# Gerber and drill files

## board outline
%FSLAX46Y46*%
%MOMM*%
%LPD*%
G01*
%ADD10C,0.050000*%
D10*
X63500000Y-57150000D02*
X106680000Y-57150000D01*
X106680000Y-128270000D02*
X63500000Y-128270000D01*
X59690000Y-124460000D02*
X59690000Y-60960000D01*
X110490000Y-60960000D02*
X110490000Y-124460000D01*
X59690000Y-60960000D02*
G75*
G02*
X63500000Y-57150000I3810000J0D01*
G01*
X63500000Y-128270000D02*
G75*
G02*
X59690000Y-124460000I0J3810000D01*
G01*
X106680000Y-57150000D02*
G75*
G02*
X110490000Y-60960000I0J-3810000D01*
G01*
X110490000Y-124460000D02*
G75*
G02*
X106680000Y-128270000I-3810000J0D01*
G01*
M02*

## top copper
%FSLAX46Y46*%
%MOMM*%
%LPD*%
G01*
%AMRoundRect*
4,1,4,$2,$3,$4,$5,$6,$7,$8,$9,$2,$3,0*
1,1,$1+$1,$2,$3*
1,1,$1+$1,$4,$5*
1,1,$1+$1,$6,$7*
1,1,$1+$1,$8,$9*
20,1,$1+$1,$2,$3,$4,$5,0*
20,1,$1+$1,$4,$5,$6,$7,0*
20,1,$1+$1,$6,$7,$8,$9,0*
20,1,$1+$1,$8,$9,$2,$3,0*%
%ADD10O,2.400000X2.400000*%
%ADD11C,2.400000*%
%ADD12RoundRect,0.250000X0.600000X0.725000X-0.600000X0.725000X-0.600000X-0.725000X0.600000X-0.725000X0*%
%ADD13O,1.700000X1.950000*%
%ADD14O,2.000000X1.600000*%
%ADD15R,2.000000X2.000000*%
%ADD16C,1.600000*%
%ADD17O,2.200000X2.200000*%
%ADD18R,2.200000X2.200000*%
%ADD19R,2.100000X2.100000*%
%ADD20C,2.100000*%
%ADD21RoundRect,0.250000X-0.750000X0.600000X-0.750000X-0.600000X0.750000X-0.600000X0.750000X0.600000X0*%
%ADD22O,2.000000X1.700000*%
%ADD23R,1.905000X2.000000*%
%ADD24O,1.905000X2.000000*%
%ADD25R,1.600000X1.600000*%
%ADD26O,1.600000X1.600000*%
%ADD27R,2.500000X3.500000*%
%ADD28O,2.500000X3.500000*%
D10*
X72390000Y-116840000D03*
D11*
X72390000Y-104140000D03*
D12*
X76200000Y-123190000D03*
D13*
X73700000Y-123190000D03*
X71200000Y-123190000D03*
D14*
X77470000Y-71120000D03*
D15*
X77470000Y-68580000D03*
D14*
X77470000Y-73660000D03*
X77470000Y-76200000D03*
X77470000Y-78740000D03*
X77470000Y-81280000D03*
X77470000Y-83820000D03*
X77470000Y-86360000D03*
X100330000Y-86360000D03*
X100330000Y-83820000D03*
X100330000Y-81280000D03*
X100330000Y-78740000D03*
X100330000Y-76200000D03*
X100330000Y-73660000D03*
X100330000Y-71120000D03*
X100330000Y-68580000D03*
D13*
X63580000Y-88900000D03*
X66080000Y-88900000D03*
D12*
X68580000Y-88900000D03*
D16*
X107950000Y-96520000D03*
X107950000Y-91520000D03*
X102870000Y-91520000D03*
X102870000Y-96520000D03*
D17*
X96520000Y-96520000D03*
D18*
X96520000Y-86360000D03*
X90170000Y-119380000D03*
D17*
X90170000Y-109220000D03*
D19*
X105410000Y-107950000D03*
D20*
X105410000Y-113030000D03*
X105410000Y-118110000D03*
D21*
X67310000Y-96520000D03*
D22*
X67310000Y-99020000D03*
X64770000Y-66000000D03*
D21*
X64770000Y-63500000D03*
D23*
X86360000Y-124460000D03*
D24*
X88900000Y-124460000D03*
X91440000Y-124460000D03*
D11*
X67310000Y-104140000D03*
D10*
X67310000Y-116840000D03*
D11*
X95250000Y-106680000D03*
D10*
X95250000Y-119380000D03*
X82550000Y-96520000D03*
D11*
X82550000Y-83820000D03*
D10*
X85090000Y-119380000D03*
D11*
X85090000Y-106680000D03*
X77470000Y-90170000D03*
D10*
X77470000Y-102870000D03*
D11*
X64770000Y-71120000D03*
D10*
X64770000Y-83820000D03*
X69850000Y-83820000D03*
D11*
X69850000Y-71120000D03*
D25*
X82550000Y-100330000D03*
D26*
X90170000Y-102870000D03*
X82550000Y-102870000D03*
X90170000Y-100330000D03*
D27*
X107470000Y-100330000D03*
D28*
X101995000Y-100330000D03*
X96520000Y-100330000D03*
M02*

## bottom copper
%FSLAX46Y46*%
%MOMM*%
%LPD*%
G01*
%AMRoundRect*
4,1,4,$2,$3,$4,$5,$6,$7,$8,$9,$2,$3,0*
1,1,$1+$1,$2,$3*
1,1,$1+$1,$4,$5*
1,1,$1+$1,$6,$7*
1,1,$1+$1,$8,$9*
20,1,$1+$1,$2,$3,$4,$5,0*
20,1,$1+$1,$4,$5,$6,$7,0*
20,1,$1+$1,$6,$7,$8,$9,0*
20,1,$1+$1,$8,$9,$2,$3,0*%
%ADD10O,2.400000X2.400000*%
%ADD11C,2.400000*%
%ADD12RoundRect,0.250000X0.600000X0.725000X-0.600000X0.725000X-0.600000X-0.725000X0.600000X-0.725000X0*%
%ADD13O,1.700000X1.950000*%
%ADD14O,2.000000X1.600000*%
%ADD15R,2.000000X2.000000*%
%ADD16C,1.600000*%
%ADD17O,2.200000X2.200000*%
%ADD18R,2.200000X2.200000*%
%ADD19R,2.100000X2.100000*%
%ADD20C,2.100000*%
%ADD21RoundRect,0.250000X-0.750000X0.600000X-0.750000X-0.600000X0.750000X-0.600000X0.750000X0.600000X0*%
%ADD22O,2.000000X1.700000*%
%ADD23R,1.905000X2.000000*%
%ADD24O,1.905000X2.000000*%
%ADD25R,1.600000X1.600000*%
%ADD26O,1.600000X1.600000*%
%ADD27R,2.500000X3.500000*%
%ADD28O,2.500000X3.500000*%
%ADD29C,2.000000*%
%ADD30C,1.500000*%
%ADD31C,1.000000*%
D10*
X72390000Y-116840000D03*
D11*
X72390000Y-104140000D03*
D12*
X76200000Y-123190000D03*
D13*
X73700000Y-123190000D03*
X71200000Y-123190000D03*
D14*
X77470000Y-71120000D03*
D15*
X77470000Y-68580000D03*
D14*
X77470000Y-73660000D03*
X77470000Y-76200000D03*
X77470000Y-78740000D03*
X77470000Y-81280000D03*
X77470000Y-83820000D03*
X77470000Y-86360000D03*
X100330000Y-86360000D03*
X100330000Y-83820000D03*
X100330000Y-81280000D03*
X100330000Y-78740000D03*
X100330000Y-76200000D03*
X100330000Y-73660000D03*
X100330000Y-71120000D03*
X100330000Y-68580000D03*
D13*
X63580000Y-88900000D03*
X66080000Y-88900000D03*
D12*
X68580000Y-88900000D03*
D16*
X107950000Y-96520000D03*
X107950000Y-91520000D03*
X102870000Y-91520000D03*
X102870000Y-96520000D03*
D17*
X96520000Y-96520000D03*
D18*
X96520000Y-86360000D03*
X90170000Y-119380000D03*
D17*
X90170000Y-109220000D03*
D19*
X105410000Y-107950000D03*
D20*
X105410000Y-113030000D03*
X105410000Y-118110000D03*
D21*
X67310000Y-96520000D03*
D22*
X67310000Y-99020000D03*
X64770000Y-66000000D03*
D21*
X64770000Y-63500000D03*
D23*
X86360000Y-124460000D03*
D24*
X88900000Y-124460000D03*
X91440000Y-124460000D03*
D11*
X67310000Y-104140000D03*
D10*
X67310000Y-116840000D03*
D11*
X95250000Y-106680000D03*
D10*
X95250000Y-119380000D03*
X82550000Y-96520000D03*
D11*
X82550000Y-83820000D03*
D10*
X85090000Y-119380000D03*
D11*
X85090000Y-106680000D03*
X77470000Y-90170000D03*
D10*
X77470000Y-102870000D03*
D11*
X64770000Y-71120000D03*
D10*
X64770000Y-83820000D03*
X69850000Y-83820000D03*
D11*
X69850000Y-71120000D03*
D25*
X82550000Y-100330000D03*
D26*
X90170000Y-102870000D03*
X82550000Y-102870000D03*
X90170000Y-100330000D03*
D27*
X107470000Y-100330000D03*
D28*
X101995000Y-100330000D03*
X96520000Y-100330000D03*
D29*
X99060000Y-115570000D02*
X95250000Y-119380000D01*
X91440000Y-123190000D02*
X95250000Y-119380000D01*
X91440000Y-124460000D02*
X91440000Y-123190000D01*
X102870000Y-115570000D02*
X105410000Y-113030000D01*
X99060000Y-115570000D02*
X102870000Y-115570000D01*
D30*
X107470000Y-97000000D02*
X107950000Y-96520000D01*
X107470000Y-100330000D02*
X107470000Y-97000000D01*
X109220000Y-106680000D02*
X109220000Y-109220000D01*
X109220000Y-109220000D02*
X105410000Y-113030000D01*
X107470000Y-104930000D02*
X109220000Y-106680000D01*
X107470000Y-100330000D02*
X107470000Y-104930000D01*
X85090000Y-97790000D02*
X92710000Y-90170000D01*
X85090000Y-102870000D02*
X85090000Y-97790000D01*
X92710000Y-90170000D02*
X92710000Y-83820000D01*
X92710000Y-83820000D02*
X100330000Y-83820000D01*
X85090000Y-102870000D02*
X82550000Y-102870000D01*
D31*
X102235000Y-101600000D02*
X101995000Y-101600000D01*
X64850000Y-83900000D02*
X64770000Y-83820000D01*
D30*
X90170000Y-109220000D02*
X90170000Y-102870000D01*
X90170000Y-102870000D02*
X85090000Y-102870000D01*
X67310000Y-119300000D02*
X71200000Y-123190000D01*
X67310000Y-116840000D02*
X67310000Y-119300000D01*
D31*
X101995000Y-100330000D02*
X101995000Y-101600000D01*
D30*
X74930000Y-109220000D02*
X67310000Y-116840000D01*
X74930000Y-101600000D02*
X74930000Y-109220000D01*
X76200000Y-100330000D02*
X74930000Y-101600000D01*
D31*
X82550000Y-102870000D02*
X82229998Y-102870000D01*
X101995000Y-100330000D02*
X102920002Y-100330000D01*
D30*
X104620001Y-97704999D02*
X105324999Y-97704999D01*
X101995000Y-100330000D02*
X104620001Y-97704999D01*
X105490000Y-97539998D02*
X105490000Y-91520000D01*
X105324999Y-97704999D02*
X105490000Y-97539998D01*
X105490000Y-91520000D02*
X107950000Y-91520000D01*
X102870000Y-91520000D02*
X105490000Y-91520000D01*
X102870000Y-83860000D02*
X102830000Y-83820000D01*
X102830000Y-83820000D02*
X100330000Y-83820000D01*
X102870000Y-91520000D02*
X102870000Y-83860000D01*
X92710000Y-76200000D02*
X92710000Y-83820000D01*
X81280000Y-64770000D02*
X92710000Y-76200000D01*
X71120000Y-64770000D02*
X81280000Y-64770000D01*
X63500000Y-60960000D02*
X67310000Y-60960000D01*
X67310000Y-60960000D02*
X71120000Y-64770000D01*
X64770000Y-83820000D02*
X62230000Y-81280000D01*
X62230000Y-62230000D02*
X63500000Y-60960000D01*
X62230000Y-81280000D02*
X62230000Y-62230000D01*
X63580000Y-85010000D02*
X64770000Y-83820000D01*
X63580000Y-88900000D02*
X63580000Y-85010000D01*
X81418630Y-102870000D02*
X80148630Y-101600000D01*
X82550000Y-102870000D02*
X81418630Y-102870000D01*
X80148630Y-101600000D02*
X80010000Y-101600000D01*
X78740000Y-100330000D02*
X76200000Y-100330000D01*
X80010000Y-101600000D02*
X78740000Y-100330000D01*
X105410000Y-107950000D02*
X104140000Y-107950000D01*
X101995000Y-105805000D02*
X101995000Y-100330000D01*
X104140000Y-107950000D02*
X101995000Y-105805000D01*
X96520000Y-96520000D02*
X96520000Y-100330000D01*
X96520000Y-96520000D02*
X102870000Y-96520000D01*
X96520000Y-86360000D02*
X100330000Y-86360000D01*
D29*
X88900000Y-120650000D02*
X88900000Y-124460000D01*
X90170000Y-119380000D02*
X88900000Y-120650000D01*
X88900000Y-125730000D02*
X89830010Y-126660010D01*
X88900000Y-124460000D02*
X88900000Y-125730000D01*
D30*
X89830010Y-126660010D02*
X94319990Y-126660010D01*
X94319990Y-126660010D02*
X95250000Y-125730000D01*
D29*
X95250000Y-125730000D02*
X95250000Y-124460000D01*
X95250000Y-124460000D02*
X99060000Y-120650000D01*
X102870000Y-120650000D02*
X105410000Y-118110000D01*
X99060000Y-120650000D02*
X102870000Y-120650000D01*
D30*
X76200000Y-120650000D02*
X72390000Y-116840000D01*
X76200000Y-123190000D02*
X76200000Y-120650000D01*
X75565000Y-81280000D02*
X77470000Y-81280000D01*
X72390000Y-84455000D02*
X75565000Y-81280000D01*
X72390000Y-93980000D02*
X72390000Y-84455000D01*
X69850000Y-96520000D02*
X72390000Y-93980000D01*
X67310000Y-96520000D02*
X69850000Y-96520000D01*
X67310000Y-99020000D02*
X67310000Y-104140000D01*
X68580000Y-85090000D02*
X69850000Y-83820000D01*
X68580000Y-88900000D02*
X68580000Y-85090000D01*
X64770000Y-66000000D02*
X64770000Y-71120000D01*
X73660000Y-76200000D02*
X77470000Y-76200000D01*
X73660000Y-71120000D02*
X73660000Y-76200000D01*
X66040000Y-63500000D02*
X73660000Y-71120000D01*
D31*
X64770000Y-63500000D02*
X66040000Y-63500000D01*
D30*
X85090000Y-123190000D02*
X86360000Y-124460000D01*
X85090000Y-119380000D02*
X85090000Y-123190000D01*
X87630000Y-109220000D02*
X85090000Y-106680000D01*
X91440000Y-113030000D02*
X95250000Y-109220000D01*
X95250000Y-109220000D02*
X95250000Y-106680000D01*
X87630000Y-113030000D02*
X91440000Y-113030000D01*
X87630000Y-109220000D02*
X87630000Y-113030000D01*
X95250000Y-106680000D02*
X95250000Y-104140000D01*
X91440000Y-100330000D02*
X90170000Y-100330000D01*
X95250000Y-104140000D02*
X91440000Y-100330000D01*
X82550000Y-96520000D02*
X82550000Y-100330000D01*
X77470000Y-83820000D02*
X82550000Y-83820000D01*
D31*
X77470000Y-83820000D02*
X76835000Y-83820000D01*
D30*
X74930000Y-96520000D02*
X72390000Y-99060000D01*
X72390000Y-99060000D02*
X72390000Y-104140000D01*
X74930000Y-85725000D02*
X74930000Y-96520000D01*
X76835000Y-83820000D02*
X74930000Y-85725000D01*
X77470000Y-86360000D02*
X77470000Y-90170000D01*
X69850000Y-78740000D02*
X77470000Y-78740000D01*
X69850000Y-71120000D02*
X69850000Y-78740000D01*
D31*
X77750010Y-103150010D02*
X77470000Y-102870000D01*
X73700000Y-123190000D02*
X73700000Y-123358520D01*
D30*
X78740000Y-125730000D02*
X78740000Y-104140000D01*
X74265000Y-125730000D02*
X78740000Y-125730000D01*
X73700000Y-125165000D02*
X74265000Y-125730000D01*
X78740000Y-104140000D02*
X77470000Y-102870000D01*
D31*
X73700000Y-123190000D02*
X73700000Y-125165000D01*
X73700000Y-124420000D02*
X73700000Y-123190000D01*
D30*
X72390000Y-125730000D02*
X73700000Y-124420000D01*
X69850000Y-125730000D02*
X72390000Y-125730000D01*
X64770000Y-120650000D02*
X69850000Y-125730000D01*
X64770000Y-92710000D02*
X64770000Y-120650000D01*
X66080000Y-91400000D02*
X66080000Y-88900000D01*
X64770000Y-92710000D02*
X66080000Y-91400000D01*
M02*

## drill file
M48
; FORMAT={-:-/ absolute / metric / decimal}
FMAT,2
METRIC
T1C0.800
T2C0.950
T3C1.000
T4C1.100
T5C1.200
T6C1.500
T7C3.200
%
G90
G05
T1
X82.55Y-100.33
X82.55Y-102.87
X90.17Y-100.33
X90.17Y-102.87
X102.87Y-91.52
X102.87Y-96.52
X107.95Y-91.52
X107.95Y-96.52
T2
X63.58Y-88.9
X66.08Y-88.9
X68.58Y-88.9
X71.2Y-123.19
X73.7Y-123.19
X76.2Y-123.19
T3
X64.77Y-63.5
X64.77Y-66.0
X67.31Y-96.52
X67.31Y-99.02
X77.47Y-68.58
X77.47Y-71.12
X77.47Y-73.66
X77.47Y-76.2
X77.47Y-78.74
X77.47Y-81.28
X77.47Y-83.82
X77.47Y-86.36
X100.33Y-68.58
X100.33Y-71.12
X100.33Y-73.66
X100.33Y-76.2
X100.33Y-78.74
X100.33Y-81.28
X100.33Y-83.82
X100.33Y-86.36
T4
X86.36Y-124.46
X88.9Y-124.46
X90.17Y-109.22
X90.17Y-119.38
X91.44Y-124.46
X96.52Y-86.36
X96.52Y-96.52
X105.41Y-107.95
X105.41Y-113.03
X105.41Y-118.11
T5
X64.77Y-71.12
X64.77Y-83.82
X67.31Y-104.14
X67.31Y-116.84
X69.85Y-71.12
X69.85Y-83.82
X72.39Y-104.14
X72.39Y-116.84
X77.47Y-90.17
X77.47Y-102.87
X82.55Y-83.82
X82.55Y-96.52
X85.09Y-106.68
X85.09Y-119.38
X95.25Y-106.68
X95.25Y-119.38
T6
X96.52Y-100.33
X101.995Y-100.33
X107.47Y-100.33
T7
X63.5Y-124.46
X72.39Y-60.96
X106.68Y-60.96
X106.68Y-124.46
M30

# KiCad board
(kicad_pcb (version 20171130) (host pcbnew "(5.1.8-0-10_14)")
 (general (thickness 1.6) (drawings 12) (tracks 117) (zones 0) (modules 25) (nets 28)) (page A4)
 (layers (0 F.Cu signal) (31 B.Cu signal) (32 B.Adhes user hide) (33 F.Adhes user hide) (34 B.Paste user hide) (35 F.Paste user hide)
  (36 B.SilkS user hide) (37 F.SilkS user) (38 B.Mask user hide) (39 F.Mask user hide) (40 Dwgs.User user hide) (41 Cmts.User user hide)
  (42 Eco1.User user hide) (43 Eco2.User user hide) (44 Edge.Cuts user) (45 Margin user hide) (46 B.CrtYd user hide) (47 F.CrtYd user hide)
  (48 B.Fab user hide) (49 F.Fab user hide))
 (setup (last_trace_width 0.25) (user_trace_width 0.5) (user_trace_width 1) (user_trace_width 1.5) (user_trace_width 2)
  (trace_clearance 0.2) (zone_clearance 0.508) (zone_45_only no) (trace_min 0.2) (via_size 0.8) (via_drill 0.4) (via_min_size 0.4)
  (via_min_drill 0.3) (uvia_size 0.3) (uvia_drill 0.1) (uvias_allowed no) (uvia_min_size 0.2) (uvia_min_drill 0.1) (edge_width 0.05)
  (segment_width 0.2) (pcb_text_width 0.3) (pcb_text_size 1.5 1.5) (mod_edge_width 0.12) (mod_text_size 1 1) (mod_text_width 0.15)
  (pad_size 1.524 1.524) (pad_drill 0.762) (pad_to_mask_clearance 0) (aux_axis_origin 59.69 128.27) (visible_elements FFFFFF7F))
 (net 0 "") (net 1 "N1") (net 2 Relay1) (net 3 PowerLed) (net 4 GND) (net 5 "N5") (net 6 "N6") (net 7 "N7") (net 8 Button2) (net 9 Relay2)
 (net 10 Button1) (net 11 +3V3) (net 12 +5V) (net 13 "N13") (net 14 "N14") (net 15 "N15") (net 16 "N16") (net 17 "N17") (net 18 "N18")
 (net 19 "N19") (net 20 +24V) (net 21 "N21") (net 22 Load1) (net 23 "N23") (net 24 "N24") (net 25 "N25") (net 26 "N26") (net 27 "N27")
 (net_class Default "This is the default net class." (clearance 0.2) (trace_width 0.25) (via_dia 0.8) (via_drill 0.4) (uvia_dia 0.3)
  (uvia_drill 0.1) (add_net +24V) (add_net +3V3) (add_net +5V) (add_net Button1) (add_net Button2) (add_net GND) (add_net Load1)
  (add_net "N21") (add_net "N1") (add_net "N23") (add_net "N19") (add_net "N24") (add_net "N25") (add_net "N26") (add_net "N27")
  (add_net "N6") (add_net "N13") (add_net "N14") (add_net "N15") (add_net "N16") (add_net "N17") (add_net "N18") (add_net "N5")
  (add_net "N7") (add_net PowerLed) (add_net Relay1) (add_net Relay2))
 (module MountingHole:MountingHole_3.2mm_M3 (layer F.Cu) (at 72.39 60.96 270)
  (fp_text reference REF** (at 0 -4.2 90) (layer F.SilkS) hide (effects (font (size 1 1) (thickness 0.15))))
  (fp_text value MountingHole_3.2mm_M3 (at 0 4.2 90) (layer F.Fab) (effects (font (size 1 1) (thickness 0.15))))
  (pad 1 np_thru_hole circle (at 0 0 270) (size 3.2 3.2) (drill 3.2) (layers *.Cu *.Mask)))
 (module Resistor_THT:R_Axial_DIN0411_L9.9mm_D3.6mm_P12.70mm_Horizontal (layer F.Cu) (at 72.39 104.14 270)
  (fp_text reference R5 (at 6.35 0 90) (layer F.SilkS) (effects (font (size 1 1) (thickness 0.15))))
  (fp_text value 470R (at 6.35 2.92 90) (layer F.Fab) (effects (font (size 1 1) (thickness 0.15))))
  (pad 2 thru_hole oval (at 12.7 0 270) (size 2.4 2.4) (drill 1.2) (layers *.Cu *.Mask) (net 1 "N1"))
  (pad 1 thru_hole circle (at 0 0 270) (size 2.4 2.4) (drill 1.2) (layers *.Cu *.Mask) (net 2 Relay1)))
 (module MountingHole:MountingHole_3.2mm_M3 (layer F.Cu) (at 106.68 124.46 270)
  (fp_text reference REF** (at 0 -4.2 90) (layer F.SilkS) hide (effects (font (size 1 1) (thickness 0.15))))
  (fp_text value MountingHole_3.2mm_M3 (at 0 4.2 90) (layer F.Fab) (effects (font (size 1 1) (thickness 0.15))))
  (pad 1 np_thru_hole circle (at 0 0 270) (size 3.2 3.2) (drill 3.2) (layers *.Cu *.Mask)))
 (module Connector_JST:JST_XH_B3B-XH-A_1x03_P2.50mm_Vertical (layer F.Cu) (at 76.2 123.19 180)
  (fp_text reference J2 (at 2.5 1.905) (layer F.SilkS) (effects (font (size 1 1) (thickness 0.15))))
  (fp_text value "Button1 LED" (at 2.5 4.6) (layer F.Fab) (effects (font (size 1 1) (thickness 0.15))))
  (pad 1 thru_hole roundrect (at 0 0 180) (size 1.7 1.95) (drill 0.95) (layers *.Cu *.Mask) (roundrect_rratio 0.1470588235294118)
   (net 1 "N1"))
  (pad 2 thru_hole oval (at 2.5 0 180) (size 1.7 1.95) (drill 0.95) (layers *.Cu *.Mask) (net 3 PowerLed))
  (pad 3 thru_hole oval (at 5 0 180) (size 1.7 1.95) (drill 0.95) (layers *.Cu *.Mask) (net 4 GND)))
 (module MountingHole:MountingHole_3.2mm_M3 (layer F.Cu) (at 63.5 124.46 270)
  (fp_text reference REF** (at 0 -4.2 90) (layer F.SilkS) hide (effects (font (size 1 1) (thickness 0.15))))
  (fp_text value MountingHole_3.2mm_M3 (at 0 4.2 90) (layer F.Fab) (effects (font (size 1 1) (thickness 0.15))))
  (pad 1 np_thru_hole circle (at 0 0 270) (size 3.2 3.2) (drill 3.2) (layers *.Cu *.Mask)))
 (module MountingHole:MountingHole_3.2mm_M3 (layer F.Cu) (at 106.68 60.96 270)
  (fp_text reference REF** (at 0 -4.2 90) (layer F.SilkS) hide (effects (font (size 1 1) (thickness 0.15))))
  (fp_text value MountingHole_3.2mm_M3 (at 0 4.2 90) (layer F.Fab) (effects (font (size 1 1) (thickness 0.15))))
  (pad 1 np_thru_hole circle (at 0 0 270) (size 3.2 3.2) (drill 3.2) (layers *.Cu *.Mask)))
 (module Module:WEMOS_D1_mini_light (layer F.Cu) (at 77.47 68.58)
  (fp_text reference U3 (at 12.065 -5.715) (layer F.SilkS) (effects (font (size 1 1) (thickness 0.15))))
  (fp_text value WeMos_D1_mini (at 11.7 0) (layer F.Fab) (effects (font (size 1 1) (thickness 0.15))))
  (pad 2 thru_hole oval (at 0 2.54) (size 2 1.6) (drill 1) (layers *.Cu *.Mask) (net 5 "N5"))
  (pad 1 thru_hole rect (at 0 0) (size 2 2) (drill 1) (layers *.Cu *.Mask) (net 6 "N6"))
  (pad 3 thru_hole oval (at 0 5.08) (size 2 1.6) (drill 1) (layers *.Cu *.Mask) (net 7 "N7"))
  (pad 4 thru_hole oval (at 0 7.62) (size 2 1.6) (drill 1) (layers *.Cu *.Mask) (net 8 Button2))
  (pad 5 thru_hole oval (at 0 10.16) (size 2 1.6) (drill 1) (layers *.Cu *.Mask) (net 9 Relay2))
  (pad 6 thru_hole oval (at 0 12.7) (size 2 1.6) (drill 1) (layers *.Cu *.Mask) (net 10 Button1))
  (pad 7 thru_hole oval (at 0 15.24) (size 2 1.6) (drill 1) (layers *.Cu *.Mask) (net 2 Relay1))
  (pad 8 thru_hole oval (at 0 17.78) (size 2 1.6) (drill 1) (layers *.Cu *.Mask) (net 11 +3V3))
  (pad 9 thru_hole oval (at 22.86 17.78) (size 2 1.6) (drill 1) (layers *.Cu *.Mask) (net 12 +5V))
  (pad 10 thru_hole oval (at 22.86 15.24) (size 2 1.6) (drill 1) (layers *.Cu *.Mask) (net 4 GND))
  (pad 11 thru_hole oval (at 22.86 12.7) (size 2 1.6) (drill 1) (layers *.Cu *.Mask) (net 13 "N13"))
  (pad 12 thru_hole oval (at 22.86 10.16) (size 2 1.6) (drill 1) (layers *.Cu *.Mask) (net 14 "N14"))
  (pad 13 thru_hole oval (at 22.86 7.62) (size 2 1.6) (drill 1) (layers *.Cu *.Mask) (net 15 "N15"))
  (pad 14 thru_hole oval (at 22.86 5.08) (size 2 1.6) (drill 1) (layers *.Cu *.Mask) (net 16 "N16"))
  (pad 15 thru_hole oval (at 22.86 2.54) (size 2 1.6) (drill 1) (layers *.Cu *.Mask) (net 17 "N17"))
  (pad 16 thru_hole oval (at 22.86 0) (size 2 1.6) (drill 1) (layers *.Cu *.Mask) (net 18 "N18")))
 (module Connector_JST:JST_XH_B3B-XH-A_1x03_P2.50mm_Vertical (layer F.Cu) (at 68.58 88.9 180)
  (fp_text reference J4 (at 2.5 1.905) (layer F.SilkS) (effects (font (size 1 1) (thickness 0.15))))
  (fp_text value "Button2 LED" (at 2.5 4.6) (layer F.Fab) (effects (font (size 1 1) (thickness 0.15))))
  (pad 3 thru_hole oval (at 5 0 180) (size 1.7 1.95) (drill 0.95) (layers *.Cu *.Mask) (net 4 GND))
  (pad 2 thru_hole oval (at 2.5 0 180) (size 1.7 1.95) (drill 0.95) (layers *.Cu *.Mask) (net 3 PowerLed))
  (pad 1 thru_hole roundrect (at 0 0 180) (size 1.7 1.95) (drill 0.95) (layers *.Cu *.Mask) (roundrect_rratio 0.1470588235294118)
   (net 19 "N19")))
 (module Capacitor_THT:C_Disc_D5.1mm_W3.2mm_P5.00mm (layer F.Cu) (at 107.95 96.52 90)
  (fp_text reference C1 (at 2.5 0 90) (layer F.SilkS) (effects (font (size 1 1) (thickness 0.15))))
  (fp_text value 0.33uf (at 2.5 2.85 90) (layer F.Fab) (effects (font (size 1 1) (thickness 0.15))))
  (pad 1 thru_hole circle (at 0 0 90) (size 1.6 1.6) (drill 0.8) (layers *.Cu *.Mask) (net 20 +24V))
  (pad 2 thru_hole circle (at 5 0 90) (size 1.6 1.6) (drill 0.8) (layers *.Cu *.Mask) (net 4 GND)))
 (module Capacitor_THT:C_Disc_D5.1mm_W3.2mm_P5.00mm (layer F.Cu) (at 102.87 96.52 90)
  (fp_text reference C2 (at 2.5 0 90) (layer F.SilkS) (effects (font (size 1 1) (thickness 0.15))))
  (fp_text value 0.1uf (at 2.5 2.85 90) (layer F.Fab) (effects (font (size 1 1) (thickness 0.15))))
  (pad 2 thru_hole circle (at 5 0 90) (size 1.6 1.6) (drill 0.8) (layers *.Cu *.Mask) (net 4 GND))
  (pad 1 thru_hole circle (at 0 0 90) (size 1.6 1.6) (drill 0.8) (layers *.Cu *.Mask) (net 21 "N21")))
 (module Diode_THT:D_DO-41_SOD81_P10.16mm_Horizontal (layer F.Cu) (at 96.52 86.36 270)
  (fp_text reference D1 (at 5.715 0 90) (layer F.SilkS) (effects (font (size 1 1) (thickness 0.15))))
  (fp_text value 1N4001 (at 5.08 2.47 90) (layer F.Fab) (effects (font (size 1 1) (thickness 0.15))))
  (pad 2 thru_hole oval (at 10.16 0 270) (size 2.2 2.2) (drill 1.1) (layers *.Cu *.Mask) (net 21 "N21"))
  (pad 1 thru_hole rect (at 0 0 270) (size 2.2 2.2) (drill 1.1) (layers *.Cu *.Mask) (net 12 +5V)))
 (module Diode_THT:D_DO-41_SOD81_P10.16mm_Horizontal (layer F.Cu) (at 90.17 119.38 90)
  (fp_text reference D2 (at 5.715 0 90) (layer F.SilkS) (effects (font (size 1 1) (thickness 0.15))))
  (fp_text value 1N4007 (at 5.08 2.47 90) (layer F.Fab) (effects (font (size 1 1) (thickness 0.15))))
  (pad 1 thru_hole rect (at 0 0 90) (size 2.2 2.2) (drill 1.1) (layers *.Cu *.Mask) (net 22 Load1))
  (pad 2 thru_hole oval (at 10.16 0 90) (size 2.2 2.2) (drill 1.1) (layers *.Cu *.Mask) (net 4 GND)))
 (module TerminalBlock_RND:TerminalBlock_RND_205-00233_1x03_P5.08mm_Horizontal (layer F.Cu) (at 105.41 107.95 270)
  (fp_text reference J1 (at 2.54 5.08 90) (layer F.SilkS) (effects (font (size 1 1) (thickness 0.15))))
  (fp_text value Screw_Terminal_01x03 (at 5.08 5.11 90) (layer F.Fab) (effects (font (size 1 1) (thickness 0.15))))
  (pad 1 thru_hole rect (at 0 0 270) (size 2.1 2.1) (drill 1.1) (layers *.Cu *.Mask) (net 4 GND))
  (pad 2 thru_hole circle (at 5.08 0 270) (size 2.1 2.1) (drill 1.1) (layers *.Cu *.Mask) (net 20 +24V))
  (pad 3 thru_hole circle (at 10.16 0 270) (size 2.1 2.1) (drill 1.1) (layers *.Cu *.Mask) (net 22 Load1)))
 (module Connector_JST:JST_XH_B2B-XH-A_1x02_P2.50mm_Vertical (layer F.Cu) (at 67.31 96.52 270)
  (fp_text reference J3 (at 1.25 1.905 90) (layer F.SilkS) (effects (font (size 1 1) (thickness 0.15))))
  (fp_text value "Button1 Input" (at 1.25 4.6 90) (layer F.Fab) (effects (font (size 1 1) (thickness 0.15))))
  (pad 1 thru_hole roundrect (at 0 0 270) (size 1.7 2) (drill 1) (layers *.Cu *.Mask) (roundrect_rratio 0.1470588235294118) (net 10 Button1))
  (pad 2 thru_hole oval (at 2.5 0 270) (size 1.7 2) (drill 1) (layers *.Cu *.Mask) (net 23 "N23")))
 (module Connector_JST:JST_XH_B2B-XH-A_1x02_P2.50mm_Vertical (layer F.Cu) (at 64.77 63.5 270)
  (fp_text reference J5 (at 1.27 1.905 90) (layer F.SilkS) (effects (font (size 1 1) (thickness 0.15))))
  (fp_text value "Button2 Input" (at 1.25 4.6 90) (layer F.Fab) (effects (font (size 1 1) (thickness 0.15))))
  (pad 2 thru_hole oval (at 2.5 0 270) (size 1.7 2) (drill 1) (layers *.Cu *.Mask) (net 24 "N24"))
  (pad 1 thru_hole roundrect (at 0 0 270) (size 1.7 2) (drill 1) (layers *.Cu *.Mask) (roundrect_rratio 0.1470588235294118) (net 8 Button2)))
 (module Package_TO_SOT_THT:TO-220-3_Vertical (layer F.Cu) (at 86.36 124.46)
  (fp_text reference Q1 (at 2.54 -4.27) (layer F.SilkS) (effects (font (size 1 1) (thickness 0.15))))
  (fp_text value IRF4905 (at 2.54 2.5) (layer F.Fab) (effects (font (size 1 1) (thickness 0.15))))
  (pad 1 thru_hole rect (at 0 0) (size 1.905 2) (drill 1.1) (layers *.Cu *.Mask) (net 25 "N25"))
  (pad 2 thru_hole oval (at 2.54 0) (size 1.905 2) (drill 1.1) (layers *.Cu *.Mask) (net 22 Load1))
  (pad 3 thru_hole oval (at 5.08 0) (size 1.905 2) (drill 1.1) (layers *.Cu *.Mask) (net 20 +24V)))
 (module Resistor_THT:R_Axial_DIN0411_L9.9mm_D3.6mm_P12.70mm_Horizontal (layer F.Cu) (at 67.31 104.14 270)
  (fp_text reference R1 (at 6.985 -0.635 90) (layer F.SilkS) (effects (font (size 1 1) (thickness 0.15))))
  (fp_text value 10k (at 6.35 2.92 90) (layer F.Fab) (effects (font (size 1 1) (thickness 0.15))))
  (pad 1 thru_hole circle (at 0 0 270) (size 2.4 2.4) (drill 1.2) (layers *.Cu *.Mask) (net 23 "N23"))
  (pad 2 thru_hole oval (at 12.7 0 270) (size 2.4 2.4) (drill 1.2) (layers *.Cu *.Mask) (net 4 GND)))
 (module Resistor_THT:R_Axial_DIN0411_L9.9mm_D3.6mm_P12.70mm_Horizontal (layer F.Cu) (at 95.25 106.68 270)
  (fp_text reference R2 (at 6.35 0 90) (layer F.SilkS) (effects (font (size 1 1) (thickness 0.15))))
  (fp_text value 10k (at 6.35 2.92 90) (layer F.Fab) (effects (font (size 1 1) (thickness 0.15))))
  (pad 1 thru_hole circle (at 0 0 270) (size 2.4 2.4) (drill 1.2) (layers *.Cu *.Mask) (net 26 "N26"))
  (pad 2 thru_hole oval (at 12.7 0 270) (size 2.4 2.4) (drill 1.2) (layers *.Cu *.Mask) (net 20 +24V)))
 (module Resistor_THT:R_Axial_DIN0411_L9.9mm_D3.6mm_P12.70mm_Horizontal (layer F.Cu) (at 82.55 83.82 270)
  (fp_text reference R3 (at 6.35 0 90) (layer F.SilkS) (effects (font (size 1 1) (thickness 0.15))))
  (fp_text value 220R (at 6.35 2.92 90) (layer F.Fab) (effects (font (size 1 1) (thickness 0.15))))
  (pad 2 thru_hole oval (at 12.7 0 270) (size 2.4 2.4) (drill 1.2) (layers *.Cu *.Mask) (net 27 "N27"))
  (pad 1 thru_hole circle (at 0 0 270) (size 2.4 2.4) (drill 1.2) (layers *.Cu *.Mask) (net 2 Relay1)))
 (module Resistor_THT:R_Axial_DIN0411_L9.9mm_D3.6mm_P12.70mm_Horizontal (layer F.Cu) (at 85.09 106.68 270)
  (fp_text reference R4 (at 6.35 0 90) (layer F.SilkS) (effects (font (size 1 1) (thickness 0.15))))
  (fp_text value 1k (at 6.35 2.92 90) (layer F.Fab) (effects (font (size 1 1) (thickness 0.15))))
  (pad 2 thru_hole oval (at 12.7 0 270) (size 2.4 2.4) (drill 1.2) (layers *.Cu *.Mask) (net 25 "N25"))
  (pad 1 thru_hole circle (at 0 0 270) (size 2.4 2.4) (drill 1.2) (layers *.Cu *.Mask) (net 26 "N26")))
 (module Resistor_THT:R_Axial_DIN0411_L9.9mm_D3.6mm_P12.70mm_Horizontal (layer F.Cu) (at 77.47 90.17 270)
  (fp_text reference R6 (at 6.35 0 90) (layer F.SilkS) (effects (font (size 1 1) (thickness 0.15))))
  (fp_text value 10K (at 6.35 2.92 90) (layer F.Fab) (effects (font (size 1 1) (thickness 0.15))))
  (pad 1 thru_hole circle (at 0 0 270) (size 2.4 2.4) (drill 1.2) (layers *.Cu *.Mask) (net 11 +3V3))
  (pad 2 thru_hole oval (at 12.7 0 270) (size 2.4 2.4) (drill 1.2) (layers *.Cu *.Mask) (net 3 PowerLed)))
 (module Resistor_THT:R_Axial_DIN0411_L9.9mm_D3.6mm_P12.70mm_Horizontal (layer F.Cu) (at 64.77 71.12 270)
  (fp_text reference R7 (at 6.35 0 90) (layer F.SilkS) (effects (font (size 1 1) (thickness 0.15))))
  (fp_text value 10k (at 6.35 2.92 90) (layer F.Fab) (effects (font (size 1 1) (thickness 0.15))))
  (pad 1 thru_hole circle (at 0 0 270) (size 2.4 2.4) (drill 1.2) (layers *.Cu *.Mask) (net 24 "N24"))
  (pad 2 thru_hole oval (at 12.7 0 270) (size 2.4 2.4) (drill 1.2) (layers *.Cu *.Mask) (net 4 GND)))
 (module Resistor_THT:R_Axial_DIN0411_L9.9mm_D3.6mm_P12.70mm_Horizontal (layer F.Cu) (at 69.85 71.12 270)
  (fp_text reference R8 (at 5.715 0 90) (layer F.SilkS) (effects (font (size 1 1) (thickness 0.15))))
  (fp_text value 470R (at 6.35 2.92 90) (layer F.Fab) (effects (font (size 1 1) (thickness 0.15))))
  (pad 2 thru_hole oval (at 12.7 0 270) (size 2.4 2.4) (drill 1.2) (layers *.Cu *.Mask) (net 19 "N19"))
  (pad 1 thru_hole circle (at 0 0 270) (size 2.4 2.4) (drill 1.2) (layers *.Cu *.Mask) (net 9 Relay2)))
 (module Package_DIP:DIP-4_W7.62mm (layer F.Cu) (at 82.55 100.33)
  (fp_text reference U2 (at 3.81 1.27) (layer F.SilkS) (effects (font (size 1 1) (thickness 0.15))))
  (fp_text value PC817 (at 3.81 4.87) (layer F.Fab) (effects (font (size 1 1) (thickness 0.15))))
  (pad 1 thru_hole rect (at 0 0) (size 1.6 1.6) (drill 0.8) (layers *.Cu *.Mask) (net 27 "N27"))
  (pad 3 thru_hole oval (at 7.62 2.54) (size 1.6 1.6) (drill 0.8) (layers *.Cu *.Mask) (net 4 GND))
  (pad 2 thru_hole oval (at 0 2.54) (size 1.6 1.6) (drill 0.8) (layers *.Cu *.Mask) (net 4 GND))
  (pad 4 thru_hole oval (at 7.62 0) (size 1.6 1.6) (drill 0.8) (layers *.Cu *.Mask) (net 26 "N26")))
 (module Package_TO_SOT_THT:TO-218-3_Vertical (layer F.Cu) (at 107.47 100.33 180)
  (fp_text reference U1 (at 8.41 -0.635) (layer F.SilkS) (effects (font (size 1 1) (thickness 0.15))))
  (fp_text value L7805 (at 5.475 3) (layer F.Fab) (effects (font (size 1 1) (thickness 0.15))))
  (pad 1 thru_hole rect (at 0 0 180) (size 2.5 3.5) (drill 1.5) (layers *.Cu *.Mask) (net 20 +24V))
  (pad 2 thru_hole oval (at 5.475 0 180) (size 2.5 3.5) (drill 1.5) (layers *.Cu *.Mask) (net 4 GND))
  (pad 3 thru_hole oval (at 10.95 0 180) (size 2.5 3.5) (drill 1.5) (layers *.Cu *.Mask) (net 21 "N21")))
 (gr_line (start 63.5 57.15) (end 106.68 57.15) (layer Edge.Cuts) (width 0.05))
 (gr_line (start 106.68 128.27) (end 63.5 128.27) (layer Edge.Cuts) (width 0.05))
 (gr_line (start 59.69 124.46) (end 59.69 60.96) (layer Edge.Cuts) (width 0.05))
 (gr_line (start 110.49 60.96) (end 110.49 124.46) (layer Edge.Cuts) (width 0.05))
 (gr_arc (start 63.5 60.96) (end 63.5 57.15) (angle -90) (layer Edge.Cuts) (width 0.05))
 (gr_arc (start 63.5 124.46) (end 59.69 124.46) (angle -90) (layer Edge.Cuts) (width 0.05))
 (gr_arc (start 106.68 60.96) (end 110.49 60.96) (angle -90) (layer Edge.Cuts) (width 0.05))
 (gr_arc (start 106.68 124.46) (end 106.68 128.27) (angle -90) (layer Edge.Cuts) (width 0.05))
 (segment (start 99.06 115.57) (end 95.25 119.38) (width 2) (layer B.Cu) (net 20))
 (segment (start 91.44 123.19) (end 95.25 119.38) (width 2) (layer B.Cu) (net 20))
 (segment (start 91.44 124.46) (end 91.44 123.19) (width 2) (layer B.Cu) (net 20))
 (segment (start 102.87 115.57) (end 105.41 113.03) (width 2) (layer B.Cu) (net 20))
 (segment (start 99.06 115.57) (end 102.87 115.57) (width 2) (layer B.Cu) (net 20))
 (segment (start 107.47 97) (end 107.95 96.52) (width 1.5) (layer B.Cu) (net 20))
 (segment (start 107.47 100.33) (end 107.47 97) (width 1.5) (layer B.Cu) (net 20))
 (segment (start 109.22 106.68) (end 109.22 109.22) (width 1.5) (layer B.Cu) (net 20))
 (segment (start 109.22 109.22) (end 105.41 113.03) (width 1.5) (layer B.Cu) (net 20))
 (segment (start 107.47 104.93) (end 109.22 106.68) (width 1.5) (layer B.Cu) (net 20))
 (segment (start 107.47 100.33) (end 107.47 104.93) (width 1.5) (layer B.Cu) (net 20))
 (segment (start 85.09 97.79) (end 92.71 90.17) (width 1.5) (layer B.Cu) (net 4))
 (segment (start 85.09 102.87) (end 85.09 97.79) (width 1.5) (layer B.Cu) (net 4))
 (segment (start 92.71 90.17) (end 92.71 83.82) (width 1.5) (layer B.Cu) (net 4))
 (segment (start 92.71 83.82) (end 100.33 83.82) (width 1.5) (layer B.Cu) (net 4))
 (segment (start 85.09 102.87) (end 82.55 102.87) (width 1.5) (layer B.Cu) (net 4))
 (segment (start 102.235 101.6) (end 101.995 101.6) (width 1) (layer B.Cu) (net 4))
 (segment (start 64.85 83.9) (end 64.77 83.82) (width 1) (layer B.Cu) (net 4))
 (segment (start 90.17 109.22) (end 90.17 102.87) (width 1.5) (layer B.Cu) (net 4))
 (segment (start 90.17 102.87) (end 85.09 102.87) (width 1.5) (layer B.Cu) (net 4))
 (segment (start 67.31 119.3) (end 71.2 123.19) (width 1.5) (layer B.Cu) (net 4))
 (segment (start 67.31 116.84) (end 67.31 119.3) (width 1.5) (layer B.Cu) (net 4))
 (segment (start 101.995 100.33) (end 101.995 101.6) (width 1) (layer B.Cu) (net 4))
 (segment (start 74.93 109.22) (end 67.31 116.84) (width 1.5) (layer B.Cu) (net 4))
 (segment (start 74.93 101.6) (end 74.93 109.22) (width 1.5) (layer B.Cu) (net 4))
 (segment (start 76.2 100.33) (end 74.93 101.6) (width 1.5) (layer B.Cu) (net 4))
 (segment (start 82.55 102.87) (end 82.229998 102.87) (width 1) (layer B.Cu) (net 4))
 (segment (start 101.995 100.33) (end 102.920002 100.33) (width 1) (layer B.Cu) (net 4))
 (segment (start 104.620001 97.704999) (end 105.324999 97.704999) (width 1.5) (layer B.Cu) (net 4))
 (segment (start 101.995 100.33) (end 104.620001 97.704999) (width 1.5) (layer B.Cu) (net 4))
 (segment (start 105.49 97.539998) (end 105.49 91.52) (width 1.5) (layer B.Cu) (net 4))
 (segment (start 105.324999 97.704999) (end 105.49 97.539998) (width 1.5) (layer B.Cu) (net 4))
 (segment (start 105.49 91.52) (end 107.95 91.52) (width 1.5) (layer B.Cu) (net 4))
 (segment (start 102.87 91.52) (end 105.49 91.52) (width 1.5) (layer B.Cu) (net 4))
 (segment (start 102.87 83.86) (end 102.83 83.82) (width 1.5) (layer B.Cu) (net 4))
 (segment (start 102.83 83.82) (end 100.33 83.82) (width 1.5) (layer B.Cu) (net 4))
 (segment (start 102.87 91.52) (end 102.87 83.86) (width 1.5) (layer B.Cu) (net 4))
 (segment (start 92.71 76.2) (end 92.71 83.82) (width 1.5) (layer B.Cu) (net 4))
 (segment (start 81.28 64.77) (end 92.71 76.2) (width 1.5) (layer B.Cu) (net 4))
 (segment (start 71.12 64.77) (end 81.28 64.77) (width 1.5) (layer B.Cu) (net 4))
 (segment (start 63.5 60.96) (end 67.31 60.96) (width 1.5) (layer B.Cu) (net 4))
 (segment (start 67.31 60.96) (end 71.12 64.77) (width 1.5) (layer B.Cu) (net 4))
 (segment (start 64.77 83.82) (end 62.23 81.28) (width 1.5) (layer B.Cu) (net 4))
 (segment (start 62.23 62.23) (end 63.5 60.96) (width 1.5) (layer B.Cu) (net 4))
 (segment (start 62.23 81.28) (end 62.23 62.23) (width 1.5) (layer B.Cu) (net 4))
 (segment (start 63.58 85.01) (end 64.77 83.82) (width 1.5) (layer B.Cu) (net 4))
 (segment (start 63.58 88.9) (end 63.58 85.01) (width 1.5) (layer B.Cu) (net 4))
 (segment (start 81.41863 102.87) (end 80.14863 101.6) (width 1.5) (layer B.Cu) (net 4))
 (segment (start 82.55 102.87) (end 81.41863 102.87) (width 1.5) (layer B.Cu) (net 4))
 (segment (start 80.14863 101.6) (end 80.01 101.6) (width 1.5) (layer B.Cu) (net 4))
 (segment (start 78.74 100.33) (end 76.2 100.33) (width 1.5) (layer B.Cu) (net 4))
 (segment (start 80.01 101.6) (end 78.74 100.33) (width 1.5) (layer B.Cu) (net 4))
 (segment (start 105.41 107.95) (end 104.14 107.95) (width 1.5) (layer B.Cu) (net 4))
 (segment (start 101.995 105.805) (end 101.995 100.33) (width 1.5) (layer B.Cu) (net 4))
 (segment (start 104.14 107.95) (end 101.995 105.805) (width 1.5) (layer B.Cu) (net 4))
 (segment (start 96.52 96.52) (end 96.52 100.33) (width 1.5) (layer B.Cu) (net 21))
 (segment (start 96.52 96.52) (end 102.87 96.52) (width 1.5) (layer B.Cu) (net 21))
 (segment (start 96.52 86.36) (end 100.33 86.36) (width 1.5) (layer B.Cu) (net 12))
 (segment (start 88.9 120.65) (end 88.9 124.46) (width 2) (layer B.Cu) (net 22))
 (segment (start 90.17 119.38) (end 88.9 120.65) (width 2) (layer B.Cu) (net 22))
 (segment (start 88.9 125.73) (end 89.83001 126.66001) (width 2) (layer B.Cu) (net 22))
 (segment (start 88.9 124.46) (end 88.9 125.73) (width 2) (layer B.Cu) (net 22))
 (segment (start 89.83001 126.66001) (end 94.31999 126.66001) (width 1.5) (layer B.Cu) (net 22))
 (segment (start 94.31999 126.66001) (end 95.25 125.73) (width 1.5) (layer B.Cu) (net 22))
 (segment (start 95.25 125.73) (end 95.25 124.46) (width 2) (layer B.Cu) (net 22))
 (segment (start 95.25 124.46) (end 99.06 120.65) (width 2) (layer B.Cu) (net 22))
 (segment (start 102.87 120.65) (end 105.41 118.11) (width 2) (layer B.Cu) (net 22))
 (segment (start 99.06 120.65) (end 102.87 120.65) (width 2) (layer B.Cu) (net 22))
 (segment (start 76.2 120.65) (end 72.39 116.84) (width 1.5) (layer B.Cu) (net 1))
 (segment (start 76.2 123.19) (end 76.2 120.65) (width 1.5) (layer B.Cu) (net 1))
 (segment (start 75.565 81.28) (end 77.47 81.28) (width 1.5) (layer B.Cu) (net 10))
 (segment (start 72.39 84.455) (end 75.565 81.28) (width 1.5) (layer B.Cu) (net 10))
 (segment (start 72.39 93.98) (end 72.39 84.455) (width 1.5) (layer B.Cu) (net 10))
 (segment (start 69.85 96.52) (end 72.39 93.98) (width 1.5) (layer B.Cu) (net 10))
 (segment (start 67.31 96.52) (end 69.85 96.52) (width 1.5) (layer B.Cu) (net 10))
 (segment (start 67.31 99.02) (end 67.31 104.14) (width 1.5) (layer B.Cu) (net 23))
 (segment (start 68.58 85.09) (end 69.85 83.82) (width 1.5) (layer B.Cu) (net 19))
 (segment (start 68.58 88.9) (end 68.58 85.09) (width 1.5) (layer B.Cu) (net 19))
 (segment (start 64.77 66) (end 64.77 71.12) (width 1.5) (layer B.Cu) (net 24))
 (segment (start 73.66 76.2) (end 77.47 76.2) (width 1.5) (layer B.Cu) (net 8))
 (segment (start 73.66 71.12) (end 73.66 76.2) (width 1.5) (layer B.Cu) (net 8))
 (segment (start 66.04 63.5) (end 73.66 71.12) (width 1.5) (layer B.Cu) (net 8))
 (segment (start 64.77 63.5) (end 66.04 63.5) (width 1) (layer B.Cu) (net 8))
 (segment (start 85.09 123.19) (end 86.36 124.46) (width 1.5) (layer B.Cu) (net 25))
 (segment (start 85.09 119.38) (end 85.09 123.19) (width 1.5) (layer B.Cu) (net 25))
 (segment (start 87.63 109.22) (end 85.09 106.68) (width 1.5) (layer B.Cu) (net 26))
 (segment (start 91.44 113.03) (end 95.25 109.22) (width 1.5) (layer B.Cu) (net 26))
 (segment (start 95.25 109.22) (end 95.25 106.68) (width 1.5) (layer B.Cu) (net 26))
 (segment (start 87.63 113.03) (end 91.44 113.03) (width 1.5) (layer B.Cu) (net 26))
 (segment (start 87.63 109.22) (end 87.63 113.03) (width 1.5) (layer B.Cu) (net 26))
 (segment (start 95.25 106.68) (end 95.25 104.14) (width 1.5) (layer B.Cu) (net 26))
 (segment (start 91.44 100.33) (end 90.17 100.33) (width 1.5) (layer B.Cu) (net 26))
 (segment (start 95.25 104.14) (end 91.44 100.33) (width 1.5) (layer B.Cu) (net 26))
 (segment (start 82.55 96.52) (end 82.55 100.33) (width 1.5) (layer B.Cu) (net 27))
 (segment (start 77.47 83.82) (end 82.55 83.82) (width 1.5) (layer B.Cu) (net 2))
 (segment (start 77.47 83.82) (end 76.835 83.82) (width 1) (layer B.Cu) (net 2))
 (segment (start 74.93 96.52) (end 72.39 99.06) (width 1.5) (layer B.Cu) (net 2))
 (segment (start 72.39 99.06) (end 72.39 104.14) (width 1.5) (layer B.Cu) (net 2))
 (segment (start 74.93 85.725) (end 74.93 96.52) (width 1.5) (layer B.Cu) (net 2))
 (segment (start 76.835 83.82) (end 74.93 85.725) (width 1.5) (layer B.Cu) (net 2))
 (segment (start 77.47 86.36) (end 77.47 90.17) (width 1.5) (layer B.Cu) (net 11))
 (segment (start 69.85 78.74) (end 77.47 78.74) (width 1.5) (layer B.Cu) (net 9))
 (segment (start 69.85 71.12) (end 69.85 78.74) (width 1.5) (layer B.Cu) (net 9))
 (segment (start 77.75001 103.15001) (end 77.47 102.87) (width 1) (layer B.Cu) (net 3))
 (segment (start 73.7 123.19) (end 73.7 123.35852) (width 1) (layer B.Cu) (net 3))
 (segment (start 78.74 125.73) (end 78.74 104.14) (width 1.5) (layer B.Cu) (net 3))
 (segment (start 74.265 125.73) (end 78.74 125.73) (width 1.5) (layer B.Cu) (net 3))
 (segment (start 73.7 125.165) (end 74.265 125.73) (width 1.5) (layer B.Cu) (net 3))
 (segment (start 78.74 104.14) (end 77.47 102.87) (width 1.5) (layer B.Cu) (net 3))
 (segment (start 73.7 123.19) (end 73.7 125.165) (width 1) (layer B.Cu) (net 3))
 (segment (start 73.7 124.42) (end 73.7 123.19) (width 1) (layer B.Cu) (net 3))
 (segment (start 72.39 125.73) (end 73.7 124.42) (width 1.5) (layer B.Cu) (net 3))
 (segment (start 69.85 125.73) (end 72.39 125.73) (width 1.5) (layer B.Cu) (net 3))
 (segment (start 64.77 120.65) (end 69.85 125.73) (width 1.5) (layer B.Cu) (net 3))
 (segment (start 64.77 92.71) (end 64.77 120.65) (width 1.5) (layer B.Cu) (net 3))
 (segment (start 66.08 91.4) (end 66.08 88.9) (width 1.5) (layer B.Cu) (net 3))
 (segment (start 64.77 92.71) (end 66.08 91.4) (width 1.5) (layer B.Cu) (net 3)))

